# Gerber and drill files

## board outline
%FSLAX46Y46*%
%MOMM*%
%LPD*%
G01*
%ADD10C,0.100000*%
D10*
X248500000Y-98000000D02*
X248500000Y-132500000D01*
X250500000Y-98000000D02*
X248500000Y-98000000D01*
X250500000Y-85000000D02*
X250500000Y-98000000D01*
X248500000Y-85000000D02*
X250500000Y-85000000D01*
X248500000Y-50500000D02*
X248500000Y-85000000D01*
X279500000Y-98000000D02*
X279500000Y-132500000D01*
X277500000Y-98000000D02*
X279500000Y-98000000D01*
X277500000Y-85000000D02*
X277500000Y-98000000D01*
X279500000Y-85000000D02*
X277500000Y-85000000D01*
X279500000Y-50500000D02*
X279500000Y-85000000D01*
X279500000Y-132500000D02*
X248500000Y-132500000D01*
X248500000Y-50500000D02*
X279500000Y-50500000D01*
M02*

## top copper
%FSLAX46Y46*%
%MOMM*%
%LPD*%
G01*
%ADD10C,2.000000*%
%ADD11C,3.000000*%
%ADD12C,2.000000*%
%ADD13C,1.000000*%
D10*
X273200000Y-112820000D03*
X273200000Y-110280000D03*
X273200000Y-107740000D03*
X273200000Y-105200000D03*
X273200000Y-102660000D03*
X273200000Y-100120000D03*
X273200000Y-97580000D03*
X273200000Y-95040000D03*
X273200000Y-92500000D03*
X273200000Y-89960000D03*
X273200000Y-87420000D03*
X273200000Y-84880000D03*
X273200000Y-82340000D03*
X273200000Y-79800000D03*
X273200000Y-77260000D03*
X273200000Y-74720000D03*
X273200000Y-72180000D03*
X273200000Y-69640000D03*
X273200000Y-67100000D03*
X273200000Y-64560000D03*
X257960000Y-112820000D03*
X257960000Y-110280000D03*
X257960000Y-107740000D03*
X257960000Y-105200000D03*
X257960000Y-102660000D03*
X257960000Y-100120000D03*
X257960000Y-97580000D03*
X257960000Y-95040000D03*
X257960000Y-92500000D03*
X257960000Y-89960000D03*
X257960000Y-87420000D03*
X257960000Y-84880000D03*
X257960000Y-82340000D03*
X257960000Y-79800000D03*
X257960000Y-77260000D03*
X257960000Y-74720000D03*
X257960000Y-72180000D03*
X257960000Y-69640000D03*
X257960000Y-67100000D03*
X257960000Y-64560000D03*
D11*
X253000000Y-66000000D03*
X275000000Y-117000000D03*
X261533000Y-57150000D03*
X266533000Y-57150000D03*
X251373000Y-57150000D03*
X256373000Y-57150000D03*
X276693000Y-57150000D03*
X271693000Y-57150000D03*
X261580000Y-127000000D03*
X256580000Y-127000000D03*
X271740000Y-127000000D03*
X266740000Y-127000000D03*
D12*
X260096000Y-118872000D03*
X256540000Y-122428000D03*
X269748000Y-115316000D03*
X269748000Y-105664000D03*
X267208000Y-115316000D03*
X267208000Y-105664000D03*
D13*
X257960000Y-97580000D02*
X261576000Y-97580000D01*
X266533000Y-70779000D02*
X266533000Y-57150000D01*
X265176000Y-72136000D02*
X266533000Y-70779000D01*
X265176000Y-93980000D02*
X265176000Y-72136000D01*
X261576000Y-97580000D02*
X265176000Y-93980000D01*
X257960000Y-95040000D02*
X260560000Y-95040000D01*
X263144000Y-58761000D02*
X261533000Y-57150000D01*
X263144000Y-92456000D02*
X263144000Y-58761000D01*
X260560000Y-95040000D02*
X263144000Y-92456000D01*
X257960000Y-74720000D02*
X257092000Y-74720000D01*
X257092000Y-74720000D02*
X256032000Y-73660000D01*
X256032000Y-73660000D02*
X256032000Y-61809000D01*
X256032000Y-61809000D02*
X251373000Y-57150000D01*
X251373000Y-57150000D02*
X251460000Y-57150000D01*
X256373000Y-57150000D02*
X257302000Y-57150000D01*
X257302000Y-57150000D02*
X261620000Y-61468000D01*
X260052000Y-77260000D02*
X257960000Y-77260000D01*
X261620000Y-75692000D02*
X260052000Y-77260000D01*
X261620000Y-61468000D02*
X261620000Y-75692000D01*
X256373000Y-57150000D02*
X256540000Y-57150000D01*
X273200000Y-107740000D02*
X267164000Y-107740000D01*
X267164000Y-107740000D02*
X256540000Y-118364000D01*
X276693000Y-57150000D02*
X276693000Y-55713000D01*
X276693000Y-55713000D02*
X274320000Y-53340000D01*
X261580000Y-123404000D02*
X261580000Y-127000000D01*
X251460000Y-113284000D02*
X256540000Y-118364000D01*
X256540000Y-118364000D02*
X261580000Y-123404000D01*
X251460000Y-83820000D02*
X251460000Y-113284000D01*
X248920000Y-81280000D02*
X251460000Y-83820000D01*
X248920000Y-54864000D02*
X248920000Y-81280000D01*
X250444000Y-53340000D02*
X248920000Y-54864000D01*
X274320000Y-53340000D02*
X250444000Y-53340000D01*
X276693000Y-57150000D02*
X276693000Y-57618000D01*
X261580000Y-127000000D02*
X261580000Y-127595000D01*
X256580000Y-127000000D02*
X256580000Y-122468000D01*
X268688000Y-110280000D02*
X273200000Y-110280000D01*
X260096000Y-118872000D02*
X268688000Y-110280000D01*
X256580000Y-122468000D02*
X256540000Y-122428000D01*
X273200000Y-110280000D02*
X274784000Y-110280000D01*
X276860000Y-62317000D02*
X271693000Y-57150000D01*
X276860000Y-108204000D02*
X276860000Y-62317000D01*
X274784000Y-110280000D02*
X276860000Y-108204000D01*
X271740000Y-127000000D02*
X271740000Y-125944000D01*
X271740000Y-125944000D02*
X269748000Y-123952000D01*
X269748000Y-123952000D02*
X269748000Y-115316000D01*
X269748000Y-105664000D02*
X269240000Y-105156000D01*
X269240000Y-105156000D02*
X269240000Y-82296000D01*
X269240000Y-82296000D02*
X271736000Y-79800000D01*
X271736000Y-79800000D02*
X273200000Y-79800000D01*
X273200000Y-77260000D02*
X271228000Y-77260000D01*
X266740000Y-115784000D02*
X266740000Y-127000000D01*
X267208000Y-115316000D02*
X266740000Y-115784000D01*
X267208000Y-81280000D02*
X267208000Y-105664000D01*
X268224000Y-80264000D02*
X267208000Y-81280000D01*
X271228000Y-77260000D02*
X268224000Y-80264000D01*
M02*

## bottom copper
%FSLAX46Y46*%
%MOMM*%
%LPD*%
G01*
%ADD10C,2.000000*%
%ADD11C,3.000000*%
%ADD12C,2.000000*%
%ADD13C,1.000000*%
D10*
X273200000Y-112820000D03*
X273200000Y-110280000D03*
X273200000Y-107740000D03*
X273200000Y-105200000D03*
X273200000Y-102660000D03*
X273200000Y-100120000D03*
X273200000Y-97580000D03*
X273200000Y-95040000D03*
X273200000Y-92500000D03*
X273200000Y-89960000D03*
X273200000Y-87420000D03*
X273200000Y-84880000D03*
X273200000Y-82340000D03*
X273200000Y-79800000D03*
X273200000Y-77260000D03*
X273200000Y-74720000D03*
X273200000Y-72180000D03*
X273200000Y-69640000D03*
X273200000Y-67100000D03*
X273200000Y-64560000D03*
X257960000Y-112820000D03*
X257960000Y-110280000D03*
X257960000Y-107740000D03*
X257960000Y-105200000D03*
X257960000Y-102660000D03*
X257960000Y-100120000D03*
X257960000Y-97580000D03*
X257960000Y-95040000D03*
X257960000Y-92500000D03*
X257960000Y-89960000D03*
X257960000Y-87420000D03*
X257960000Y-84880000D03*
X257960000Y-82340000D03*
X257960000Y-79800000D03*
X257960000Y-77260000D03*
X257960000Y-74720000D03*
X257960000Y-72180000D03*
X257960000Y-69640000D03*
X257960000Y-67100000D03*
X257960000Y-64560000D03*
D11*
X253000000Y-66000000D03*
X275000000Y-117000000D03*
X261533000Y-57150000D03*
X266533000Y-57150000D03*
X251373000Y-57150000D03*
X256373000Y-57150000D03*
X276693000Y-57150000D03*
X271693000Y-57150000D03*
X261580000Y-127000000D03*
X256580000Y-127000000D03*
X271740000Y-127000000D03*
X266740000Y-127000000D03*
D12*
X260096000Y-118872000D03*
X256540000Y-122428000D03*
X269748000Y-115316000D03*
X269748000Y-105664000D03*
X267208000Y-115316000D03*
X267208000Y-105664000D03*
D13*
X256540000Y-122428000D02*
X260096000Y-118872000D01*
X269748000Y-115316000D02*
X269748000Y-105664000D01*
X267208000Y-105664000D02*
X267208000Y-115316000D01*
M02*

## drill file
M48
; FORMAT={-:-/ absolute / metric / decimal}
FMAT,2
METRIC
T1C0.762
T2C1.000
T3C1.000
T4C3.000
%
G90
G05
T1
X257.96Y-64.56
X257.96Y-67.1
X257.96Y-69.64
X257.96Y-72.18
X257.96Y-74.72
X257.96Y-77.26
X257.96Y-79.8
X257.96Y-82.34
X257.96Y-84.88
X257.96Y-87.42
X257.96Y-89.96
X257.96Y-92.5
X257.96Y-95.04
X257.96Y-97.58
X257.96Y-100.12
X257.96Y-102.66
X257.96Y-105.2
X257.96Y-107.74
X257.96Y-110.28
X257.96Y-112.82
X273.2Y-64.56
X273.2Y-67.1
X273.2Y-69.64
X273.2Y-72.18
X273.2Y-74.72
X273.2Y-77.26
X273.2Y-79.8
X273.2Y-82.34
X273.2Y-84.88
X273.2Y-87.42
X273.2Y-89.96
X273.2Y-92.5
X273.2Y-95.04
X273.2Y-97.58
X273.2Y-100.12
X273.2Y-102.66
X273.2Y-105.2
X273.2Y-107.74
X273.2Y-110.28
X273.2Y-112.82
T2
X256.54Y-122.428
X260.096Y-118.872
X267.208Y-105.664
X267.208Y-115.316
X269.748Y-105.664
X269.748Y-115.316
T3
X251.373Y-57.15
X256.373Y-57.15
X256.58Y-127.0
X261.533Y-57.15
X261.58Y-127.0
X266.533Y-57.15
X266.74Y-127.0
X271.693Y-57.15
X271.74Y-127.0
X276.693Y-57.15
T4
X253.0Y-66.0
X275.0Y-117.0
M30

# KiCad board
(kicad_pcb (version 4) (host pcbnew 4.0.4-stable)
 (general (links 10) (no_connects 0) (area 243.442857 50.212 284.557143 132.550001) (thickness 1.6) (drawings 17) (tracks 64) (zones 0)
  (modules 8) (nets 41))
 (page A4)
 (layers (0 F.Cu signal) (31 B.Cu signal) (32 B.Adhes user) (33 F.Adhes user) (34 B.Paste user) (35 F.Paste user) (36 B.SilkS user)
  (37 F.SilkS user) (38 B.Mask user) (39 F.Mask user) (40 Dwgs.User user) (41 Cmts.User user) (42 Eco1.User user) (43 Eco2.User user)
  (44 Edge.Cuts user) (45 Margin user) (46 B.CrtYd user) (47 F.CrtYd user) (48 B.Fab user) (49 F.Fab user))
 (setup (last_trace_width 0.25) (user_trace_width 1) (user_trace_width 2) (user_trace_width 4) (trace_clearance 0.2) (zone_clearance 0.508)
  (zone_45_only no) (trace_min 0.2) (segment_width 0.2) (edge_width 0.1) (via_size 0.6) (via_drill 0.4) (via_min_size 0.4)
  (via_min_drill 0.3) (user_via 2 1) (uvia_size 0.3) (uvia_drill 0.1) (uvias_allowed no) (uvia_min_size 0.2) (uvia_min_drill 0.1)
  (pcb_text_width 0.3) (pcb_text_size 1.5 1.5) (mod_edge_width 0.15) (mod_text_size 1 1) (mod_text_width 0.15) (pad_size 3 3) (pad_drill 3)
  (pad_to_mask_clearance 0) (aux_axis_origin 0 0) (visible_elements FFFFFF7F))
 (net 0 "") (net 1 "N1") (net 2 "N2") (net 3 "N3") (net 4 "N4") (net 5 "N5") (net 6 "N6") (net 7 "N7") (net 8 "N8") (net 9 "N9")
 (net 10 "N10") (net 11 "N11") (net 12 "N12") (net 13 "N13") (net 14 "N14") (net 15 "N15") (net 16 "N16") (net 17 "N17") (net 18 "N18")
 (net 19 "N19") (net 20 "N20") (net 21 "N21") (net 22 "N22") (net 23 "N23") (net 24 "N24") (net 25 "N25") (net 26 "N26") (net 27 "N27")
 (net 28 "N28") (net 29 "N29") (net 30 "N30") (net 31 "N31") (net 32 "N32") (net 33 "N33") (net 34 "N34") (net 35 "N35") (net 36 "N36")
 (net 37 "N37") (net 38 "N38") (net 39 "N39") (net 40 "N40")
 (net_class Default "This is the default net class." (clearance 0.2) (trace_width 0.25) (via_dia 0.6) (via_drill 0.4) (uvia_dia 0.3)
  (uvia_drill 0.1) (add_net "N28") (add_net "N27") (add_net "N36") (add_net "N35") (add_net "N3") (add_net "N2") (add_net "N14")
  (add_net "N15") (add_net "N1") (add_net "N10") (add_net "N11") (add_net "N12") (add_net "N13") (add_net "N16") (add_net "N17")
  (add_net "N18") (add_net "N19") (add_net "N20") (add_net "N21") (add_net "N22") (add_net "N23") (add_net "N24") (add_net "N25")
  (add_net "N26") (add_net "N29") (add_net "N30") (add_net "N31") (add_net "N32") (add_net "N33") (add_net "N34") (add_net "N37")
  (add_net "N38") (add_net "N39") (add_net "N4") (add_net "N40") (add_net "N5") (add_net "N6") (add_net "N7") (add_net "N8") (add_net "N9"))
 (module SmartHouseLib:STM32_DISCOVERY (layer B.Cu) (at 260.5 92.5)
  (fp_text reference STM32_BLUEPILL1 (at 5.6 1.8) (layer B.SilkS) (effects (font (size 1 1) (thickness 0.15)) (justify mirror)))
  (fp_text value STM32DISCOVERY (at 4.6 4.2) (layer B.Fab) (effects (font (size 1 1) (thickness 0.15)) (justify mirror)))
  (pad 1 thru_hole circle (at 12.7 20.32) (size 2 2) (drill 0.762) (layers *.Cu *.Mask) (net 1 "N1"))
  (pad 2 thru_hole circle (at 12.7 17.78) (size 2 2) (drill 0.762) (layers *.Cu *.Mask) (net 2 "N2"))
  (pad 3 thru_hole circle (at 12.7 15.24) (size 2 2) (drill 0.762) (layers *.Cu *.Mask) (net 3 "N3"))
  (pad 4 thru_hole circle (at 12.7 12.7) (size 2 2) (drill 0.762) (layers *.Cu *.Mask) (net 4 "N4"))
  (pad 5 thru_hole circle (at 12.7 10.16) (size 2 2) (drill 0.762) (layers *.Cu *.Mask) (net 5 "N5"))
  (pad 6 thru_hole circle (at 12.7 7.62) (size 2 2) (drill 0.762) (layers *.Cu *.Mask) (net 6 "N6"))
  (pad 7 thru_hole circle (at 12.7 5.08) (size 2 2) (drill 0.762) (layers *.Cu *.Mask) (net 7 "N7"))
  (pad 8 thru_hole circle (at 12.7 2.54) (size 2 2) (drill 0.762) (layers *.Cu *.Mask) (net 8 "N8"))
  (pad 9 thru_hole circle (at 12.7 0) (size 2 2) (drill 0.762) (layers *.Cu *.Mask) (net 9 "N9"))
  (pad 10 thru_hole circle (at 12.7 -2.54) (size 2 2) (drill 0.762) (layers *.Cu *.Mask) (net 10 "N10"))
  (pad 11 thru_hole circle (at 12.7 -5.08) (size 2 2) (drill 0.762) (layers *.Cu *.Mask) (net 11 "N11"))
  (pad 12 thru_hole circle (at 12.7 -7.62) (size 2 2) (drill 0.762) (layers *.Cu *.Mask) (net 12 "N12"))
  (pad 13 thru_hole circle (at 12.7 -10.16) (size 2 2) (drill 0.762) (layers *.Cu *.Mask) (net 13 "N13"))
  (pad 14 thru_hole circle (at 12.7 -12.7) (size 2 2) (drill 0.762) (layers *.Cu *.Mask) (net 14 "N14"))
  (pad 15 thru_hole circle (at 12.7 -15.24) (size 2 2) (drill 0.762) (layers *.Cu *.Mask) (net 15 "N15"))
  (pad 16 thru_hole circle (at 12.7 -17.78) (size 2 2) (drill 0.762) (layers *.Cu *.Mask) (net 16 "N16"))
  (pad 17 thru_hole circle (at 12.7 -20.32) (size 2 2) (drill 0.762) (layers *.Cu *.Mask) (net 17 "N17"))
  (pad 18 thru_hole circle (at 12.7 -22.86) (size 2 2) (drill 0.762) (layers *.Cu *.Mask) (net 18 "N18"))
  (pad 19 thru_hole circle (at 12.7 -25.4) (size 2 2) (drill 0.762) (layers *.Cu *.Mask) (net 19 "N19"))
  (pad 20 thru_hole circle (at 12.7 -27.94) (size 2 2) (drill 0.762) (layers *.Cu *.Mask) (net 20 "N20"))
  (pad 21 thru_hole circle (at -2.54 20.32) (size 2 2) (drill 0.762) (layers *.Cu *.Mask) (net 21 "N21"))
  (pad 22 thru_hole circle (at -2.54 17.78) (size 2 2) (drill 0.762) (layers *.Cu *.Mask) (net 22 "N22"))
  (pad 23 thru_hole circle (at -2.54 15.24) (size 2 2) (drill 0.762) (layers *.Cu *.Mask) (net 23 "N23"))
  (pad 24 thru_hole circle (at -2.54 12.7) (size 2 2) (drill 0.762) (layers *.Cu *.Mask) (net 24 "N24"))
  (pad 25 thru_hole circle (at -2.54 10.16) (size 2 2) (drill 0.762) (layers *.Cu *.Mask) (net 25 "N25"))
  (pad 26 thru_hole circle (at -2.54 7.62) (size 2 2) (drill 0.762) (layers *.Cu *.Mask) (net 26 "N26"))
  (pad 27 thru_hole circle (at -2.54 5.08) (size 2 2) (drill 0.762) (layers *.Cu *.Mask) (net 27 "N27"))
  (pad 28 thru_hole circle (at -2.54 2.54) (size 2 2) (drill 0.762) (layers *.Cu *.Mask) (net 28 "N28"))
  (pad 29 thru_hole circle (at -2.54 0) (size 2 2) (drill 0.762) (layers *.Cu *.Mask) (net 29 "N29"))
  (pad 30 thru_hole circle (at -2.54 -2.54) (size 2 2) (drill 0.762) (layers *.Cu *.Mask) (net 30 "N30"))
  (pad 31 thru_hole circle (at -2.54 -5.08) (size 2 2) (drill 0.762) (layers *.Cu *.Mask) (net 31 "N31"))
  (pad 32 thru_hole circle (at -2.54 -7.62) (size 2 2) (drill 0.762) (layers *.Cu *.Mask) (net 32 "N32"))
  (pad 33 thru_hole circle (at -2.54 -10.16) (size 2 2) (drill 0.762) (layers *.Cu *.Mask) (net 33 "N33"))
  (pad 34 thru_hole circle (at -2.54 -12.7) (size 2 2) (drill 0.762) (layers *.Cu *.Mask) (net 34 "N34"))
  (pad 35 thru_hole circle (at -2.54 -15.24) (size 2 2) (drill 0.762) (layers *.Cu *.Mask) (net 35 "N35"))
  (pad 36 thru_hole circle (at -2.54 -17.78) (size 2 2) (drill 0.762) (layers *.Cu *.Mask) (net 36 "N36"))
  (pad 37 thru_hole circle (at -2.54 -20.32) (size 2 2) (drill 0.762) (layers *.Cu *.Mask) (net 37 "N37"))
  (pad 38 thru_hole circle (at -2.54 -22.86) (size 2 2) (drill 0.762) (layers *.Cu *.Mask) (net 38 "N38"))
  (pad 39 thru_hole circle (at -2.54 -25.4) (size 2 2) (drill 0.762) (layers *.Cu *.Mask) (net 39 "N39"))
  (pad 40 thru_hole circle (at -2.54 -27.94) (size 2 2) (drill 0.762) (layers *.Cu *.Mask) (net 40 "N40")))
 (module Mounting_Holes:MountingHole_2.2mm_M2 (layer F.Cu) (at 253 66)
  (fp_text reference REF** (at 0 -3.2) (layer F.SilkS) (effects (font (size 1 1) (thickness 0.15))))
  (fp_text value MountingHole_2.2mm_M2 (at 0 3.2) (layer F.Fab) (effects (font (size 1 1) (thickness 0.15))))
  (pad 1 thru_hole circle (at 0 0) (size 3 3) (drill 3) (layers *.Cu *.Mask)))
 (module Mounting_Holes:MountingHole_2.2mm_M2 (layer F.Cu) (at 275 117)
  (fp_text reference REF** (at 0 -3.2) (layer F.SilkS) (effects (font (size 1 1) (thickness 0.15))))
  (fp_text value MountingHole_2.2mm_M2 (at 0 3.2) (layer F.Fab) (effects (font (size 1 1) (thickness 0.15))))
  (pad 1 thru_hole circle (at 0 0) (size 3 3) (drill 3) (layers *.Cu *.Mask)))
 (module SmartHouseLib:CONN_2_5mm (layer B.Cu) (at 264.033 57.15)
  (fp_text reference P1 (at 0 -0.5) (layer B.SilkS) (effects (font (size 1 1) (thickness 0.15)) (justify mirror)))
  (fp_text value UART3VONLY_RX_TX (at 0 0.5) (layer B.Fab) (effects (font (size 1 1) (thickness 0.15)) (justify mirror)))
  (pad 1 thru_hole circle (at -2.5 0) (size 3 3) (drill 1) (layers *.Cu *.Mask) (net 28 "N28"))
  (pad 2 thru_hole circle (at 2.5 0) (size 3 3) (drill 1) (layers *.Cu *.Mask) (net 27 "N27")))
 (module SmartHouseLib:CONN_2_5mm (layer B.Cu) (at 253.873 57.15)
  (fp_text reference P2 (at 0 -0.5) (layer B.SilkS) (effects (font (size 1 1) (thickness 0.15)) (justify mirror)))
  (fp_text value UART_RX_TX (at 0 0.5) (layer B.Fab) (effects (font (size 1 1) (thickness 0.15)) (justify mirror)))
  (pad 1 thru_hole circle (at -2.5 0) (size 3 3) (drill 1) (layers *.Cu *.Mask) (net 36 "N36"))
  (pad 2 thru_hole circle (at 2.5 0) (size 3 3) (drill 1) (layers *.Cu *.Mask) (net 35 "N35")))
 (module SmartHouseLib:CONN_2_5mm (layer B.Cu) (at 274.193 57.15 180)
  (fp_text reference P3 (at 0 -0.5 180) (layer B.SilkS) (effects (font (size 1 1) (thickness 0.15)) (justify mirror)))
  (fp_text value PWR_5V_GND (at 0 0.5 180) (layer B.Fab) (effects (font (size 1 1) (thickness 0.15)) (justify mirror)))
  (pad 1 thru_hole circle (at -2.5 0 180) (size 3 3) (drill 1) (layers *.Cu *.Mask) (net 3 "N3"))
  (pad 2 thru_hole circle (at 2.5 0 180) (size 3 3) (drill 1) (layers *.Cu *.Mask) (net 2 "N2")))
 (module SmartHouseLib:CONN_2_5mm (layer B.Cu) (at 259.08 127 180)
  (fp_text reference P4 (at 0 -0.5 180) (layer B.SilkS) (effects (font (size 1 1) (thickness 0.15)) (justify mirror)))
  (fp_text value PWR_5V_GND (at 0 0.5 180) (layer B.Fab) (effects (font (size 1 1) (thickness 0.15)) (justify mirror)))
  (pad 1 thru_hole circle (at -2.5 0 180) (size 3 3) (drill 1) (layers *.Cu *.Mask) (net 3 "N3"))
  (pad 2 thru_hole circle (at 2.5 0 180) (size 3 3) (drill 1) (layers *.Cu *.Mask) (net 2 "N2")))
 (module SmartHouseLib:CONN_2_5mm (layer B.Cu) (at 269.24 127 180)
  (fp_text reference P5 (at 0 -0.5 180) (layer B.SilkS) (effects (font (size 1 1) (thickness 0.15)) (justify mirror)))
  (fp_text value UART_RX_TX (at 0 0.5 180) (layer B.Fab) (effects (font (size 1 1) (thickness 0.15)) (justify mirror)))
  (pad 1 thru_hole circle (at -2.5 0 180) (size 3 3) (drill 1) (layers *.Cu *.Mask) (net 14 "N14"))
  (pad 2 thru_hole circle (at 2.5 0 180) (size 3 3) (drill 1) (layers *.Cu *.Mask) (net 15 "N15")))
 (gr_line (start 248.5 98) (end 248.5 132.5) (angle 90) (layer Edge.Cuts) (width 0.1))
 (gr_line (start 250.5 98) (end 248.5 98) (angle 90) (layer Edge.Cuts) (width 0.1))
 (gr_line (start 250.5 85) (end 250.5 98) (angle 90) (layer Edge.Cuts) (width 0.1))
 (gr_line (start 248.5 85) (end 250.5 85) (angle 90) (layer Edge.Cuts) (width 0.1))
 (gr_line (start 248.5 50.5) (end 248.5 85) (angle 90) (layer Edge.Cuts) (width 0.1))
 (gr_line (start 279.5 98) (end 279.5 132.5) (angle 90) (layer Edge.Cuts) (width 0.1))
 (gr_line (start 277.5 98) (end 279.5 98) (angle 90) (layer Edge.Cuts) (width 0.1))
 (gr_line (start 277.5 85) (end 277.5 98) (angle 90) (layer Edge.Cuts) (width 0.1))
 (gr_line (start 279.5 85) (end 277.5 85) (angle 90) (layer Edge.Cuts) (width 0.1))
 (gr_line (start 279.5 50.5) (end 279.5 85) (angle 90) (layer Edge.Cuts) (width 0.1))
 (gr_line (start 279.5 132.5) (end 248.5 132.5) (angle 90) (layer Edge.Cuts) (width 0.1))
 (gr_line (start 248.5 50.5) (end 279.5 50.5) (angle 90) (layer Edge.Cuts) (width 0.1))
 (segment (start 257.96 97.58) (end 261.576 97.58) (width 1) (layer F.Cu) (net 27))
 (segment (start 266.533 70.779) (end 266.533 57.15) (width 1) (layer F.Cu) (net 27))
 (segment (start 265.176 72.136) (end 266.533 70.779) (width 1) (layer F.Cu) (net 27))
 (segment (start 265.176 93.98) (end 265.176 72.136) (width 1) (layer F.Cu) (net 27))
 (segment (start 261.576 97.58) (end 265.176 93.98) (width 1) (layer F.Cu) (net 27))
 (segment (start 257.96 95.04) (end 260.56 95.04) (width 1) (layer F.Cu) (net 28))
 (segment (start 263.144 58.761) (end 261.533 57.15) (width 1) (layer F.Cu) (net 28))
 (segment (start 263.144 92.456) (end 263.144 58.761) (width 1) (layer F.Cu) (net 28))
 (segment (start 260.56 95.04) (end 263.144 92.456) (width 1) (layer F.Cu) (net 28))
 (segment (start 257.96 74.72) (end 257.092 74.72) (width 1) (layer F.Cu) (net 36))
 (segment (start 257.092 74.72) (end 256.032 73.66) (width 1) (layer F.Cu) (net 36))
 (segment (start 256.032 73.66) (end 256.032 61.809) (width 1) (layer F.Cu) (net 36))
 (segment (start 256.032 61.809) (end 251.373 57.15) (width 1) (layer F.Cu) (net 36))
 (segment (start 251.373 57.15) (end 251.46 57.15) (width 1) (layer F.Cu) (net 36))
 (segment (start 256.373 57.15) (end 257.302 57.15) (width 1) (layer F.Cu) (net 35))
 (segment (start 257.302 57.15) (end 261.62 61.468) (width 1) (layer F.Cu) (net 35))
 (segment (start 260.052 77.26) (end 257.96 77.26) (width 1) (layer F.Cu) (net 35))
 (segment (start 261.62 75.692) (end 260.052 77.26) (width 1) (layer F.Cu) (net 35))
 (segment (start 261.62 61.468) (end 261.62 75.692) (width 1) (layer F.Cu) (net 35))
 (segment (start 256.373 57.15) (end 256.54 57.15) (width 1) (layer F.Cu) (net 35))
 (segment (start 273.2 107.74) (end 267.164 107.74) (width 1) (layer F.Cu) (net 3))
 (segment (start 267.164 107.74) (end 256.54 118.364) (width 1) (layer F.Cu) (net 3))
 (segment (start 276.693 57.15) (end 276.693 55.713) (width 1) (layer F.Cu) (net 3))
 (segment (start 276.693 55.713) (end 274.32 53.34) (width 1) (layer F.Cu) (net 3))
 (segment (start 261.58 123.404) (end 261.58 127) (width 1) (layer F.Cu) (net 3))
 (segment (start 251.46 113.284) (end 256.54 118.364) (width 1) (layer F.Cu) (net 3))
 (segment (start 256.54 118.364) (end 261.58 123.404) (width 1) (layer F.Cu) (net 3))
 (segment (start 251.46 83.82) (end 251.46 113.284) (width 1) (layer F.Cu) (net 3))
 (segment (start 248.92 81.28) (end 251.46 83.82) (width 1) (layer F.Cu) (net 3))
 (segment (start 248.92 54.864) (end 248.92 81.28) (width 1) (layer F.Cu) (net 3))
 (segment (start 250.444 53.34) (end 248.92 54.864) (width 1) (layer F.Cu) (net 3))
 (segment (start 274.32 53.34) (end 250.444 53.34) (width 1) (layer F.Cu) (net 3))
 (segment (start 276.693 57.15) (end 276.693 57.618) (width 1) (layer F.Cu) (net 3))
 (segment (start 261.58 127) (end 261.58 127.595) (width 1) (layer F.Cu) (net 3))
 (segment (start 256.58 127) (end 256.58 122.468) (width 1) (layer F.Cu) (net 2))
 (segment (start 268.688 110.28) (end 273.2 110.28) (width 1) (layer F.Cu) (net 2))
 (segment (start 260.096 118.872) (end 268.688 110.28) (width 1) (layer F.Cu) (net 2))
 (via (at 260.096 118.872) (size 2) (drill 1) (layers F.Cu B.Cu) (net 2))
 (segment (start 256.54 122.428) (end 260.096 118.872) (width 1) (layer B.Cu) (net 2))
 (via (at 256.54 122.428) (size 2) (drill 1) (layers F.Cu B.Cu) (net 2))
 (segment (start 256.58 122.468) (end 256.54 122.428) (width 1) (layer F.Cu) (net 2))
 (segment (start 273.2 110.28) (end 274.784 110.28) (width 1) (layer F.Cu) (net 2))
 (segment (start 276.86 62.317) (end 271.693 57.15) (width 1) (layer F.Cu) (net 2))
 (segment (start 276.86 108.204) (end 276.86 62.317) (width 1) (layer F.Cu) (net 2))
 (segment (start 274.784 110.28) (end 276.86 108.204) (width 1) (layer F.Cu) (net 2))
 (segment (start 271.74 127) (end 271.74 125.944) (width 1) (layer F.Cu) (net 14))
 (segment (start 271.74 125.944) (end 269.748 123.952) (width 1) (layer F.Cu) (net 14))
 (segment (start 269.748 123.952) (end 269.748 115.316) (width 1) (layer F.Cu) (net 14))
 (via (at 269.748 115.316) (size 2) (drill 1) (layers F.Cu B.Cu) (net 14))
 (segment (start 269.748 115.316) (end 269.748 105.664) (width 1) (layer B.Cu) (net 14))
 (via (at 269.748 105.664) (size 2) (drill 1) (layers F.Cu B.Cu) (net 14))
 (segment (start 269.748 105.664) (end 269.24 105.156) (width 1) (layer F.Cu) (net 14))
 (segment (start 269.24 105.156) (end 269.24 82.296) (width 1) (layer F.Cu) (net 14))
 (segment (start 269.24 82.296) (end 271.736 79.8) (width 1) (layer F.Cu) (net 14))
 (segment (start 271.736 79.8) (end 273.2 79.8) (width 1) (layer F.Cu) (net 14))
 (segment (start 273.2 77.26) (end 271.228 77.26) (width 1) (layer F.Cu) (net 15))
 (segment (start 266.74 115.784) (end 266.74 127) (width 1) (layer F.Cu) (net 15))
 (segment (start 267.208 115.316) (end 266.74 115.784) (width 1) (layer F.Cu) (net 15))
 (via (at 267.208 115.316) (size 2) (drill 1) (layers F.Cu B.Cu) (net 15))
 (segment (start 267.208 105.664) (end 267.208 115.316) (width 1) (layer B.Cu) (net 15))
 (via (at 267.208 105.664) (size 2) (drill 1) (layers F.Cu B.Cu) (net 15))
 (segment (start 267.208 81.28) (end 267.208 105.664) (width 1) (layer F.Cu) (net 15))
 (segment (start 268.224 80.264) (end 267.208 81.28) (width 1) (layer F.Cu) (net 15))
 (segment (start 271.228 77.26) (end 268.224 80.264) (width 1) (layer F.Cu) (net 15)))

